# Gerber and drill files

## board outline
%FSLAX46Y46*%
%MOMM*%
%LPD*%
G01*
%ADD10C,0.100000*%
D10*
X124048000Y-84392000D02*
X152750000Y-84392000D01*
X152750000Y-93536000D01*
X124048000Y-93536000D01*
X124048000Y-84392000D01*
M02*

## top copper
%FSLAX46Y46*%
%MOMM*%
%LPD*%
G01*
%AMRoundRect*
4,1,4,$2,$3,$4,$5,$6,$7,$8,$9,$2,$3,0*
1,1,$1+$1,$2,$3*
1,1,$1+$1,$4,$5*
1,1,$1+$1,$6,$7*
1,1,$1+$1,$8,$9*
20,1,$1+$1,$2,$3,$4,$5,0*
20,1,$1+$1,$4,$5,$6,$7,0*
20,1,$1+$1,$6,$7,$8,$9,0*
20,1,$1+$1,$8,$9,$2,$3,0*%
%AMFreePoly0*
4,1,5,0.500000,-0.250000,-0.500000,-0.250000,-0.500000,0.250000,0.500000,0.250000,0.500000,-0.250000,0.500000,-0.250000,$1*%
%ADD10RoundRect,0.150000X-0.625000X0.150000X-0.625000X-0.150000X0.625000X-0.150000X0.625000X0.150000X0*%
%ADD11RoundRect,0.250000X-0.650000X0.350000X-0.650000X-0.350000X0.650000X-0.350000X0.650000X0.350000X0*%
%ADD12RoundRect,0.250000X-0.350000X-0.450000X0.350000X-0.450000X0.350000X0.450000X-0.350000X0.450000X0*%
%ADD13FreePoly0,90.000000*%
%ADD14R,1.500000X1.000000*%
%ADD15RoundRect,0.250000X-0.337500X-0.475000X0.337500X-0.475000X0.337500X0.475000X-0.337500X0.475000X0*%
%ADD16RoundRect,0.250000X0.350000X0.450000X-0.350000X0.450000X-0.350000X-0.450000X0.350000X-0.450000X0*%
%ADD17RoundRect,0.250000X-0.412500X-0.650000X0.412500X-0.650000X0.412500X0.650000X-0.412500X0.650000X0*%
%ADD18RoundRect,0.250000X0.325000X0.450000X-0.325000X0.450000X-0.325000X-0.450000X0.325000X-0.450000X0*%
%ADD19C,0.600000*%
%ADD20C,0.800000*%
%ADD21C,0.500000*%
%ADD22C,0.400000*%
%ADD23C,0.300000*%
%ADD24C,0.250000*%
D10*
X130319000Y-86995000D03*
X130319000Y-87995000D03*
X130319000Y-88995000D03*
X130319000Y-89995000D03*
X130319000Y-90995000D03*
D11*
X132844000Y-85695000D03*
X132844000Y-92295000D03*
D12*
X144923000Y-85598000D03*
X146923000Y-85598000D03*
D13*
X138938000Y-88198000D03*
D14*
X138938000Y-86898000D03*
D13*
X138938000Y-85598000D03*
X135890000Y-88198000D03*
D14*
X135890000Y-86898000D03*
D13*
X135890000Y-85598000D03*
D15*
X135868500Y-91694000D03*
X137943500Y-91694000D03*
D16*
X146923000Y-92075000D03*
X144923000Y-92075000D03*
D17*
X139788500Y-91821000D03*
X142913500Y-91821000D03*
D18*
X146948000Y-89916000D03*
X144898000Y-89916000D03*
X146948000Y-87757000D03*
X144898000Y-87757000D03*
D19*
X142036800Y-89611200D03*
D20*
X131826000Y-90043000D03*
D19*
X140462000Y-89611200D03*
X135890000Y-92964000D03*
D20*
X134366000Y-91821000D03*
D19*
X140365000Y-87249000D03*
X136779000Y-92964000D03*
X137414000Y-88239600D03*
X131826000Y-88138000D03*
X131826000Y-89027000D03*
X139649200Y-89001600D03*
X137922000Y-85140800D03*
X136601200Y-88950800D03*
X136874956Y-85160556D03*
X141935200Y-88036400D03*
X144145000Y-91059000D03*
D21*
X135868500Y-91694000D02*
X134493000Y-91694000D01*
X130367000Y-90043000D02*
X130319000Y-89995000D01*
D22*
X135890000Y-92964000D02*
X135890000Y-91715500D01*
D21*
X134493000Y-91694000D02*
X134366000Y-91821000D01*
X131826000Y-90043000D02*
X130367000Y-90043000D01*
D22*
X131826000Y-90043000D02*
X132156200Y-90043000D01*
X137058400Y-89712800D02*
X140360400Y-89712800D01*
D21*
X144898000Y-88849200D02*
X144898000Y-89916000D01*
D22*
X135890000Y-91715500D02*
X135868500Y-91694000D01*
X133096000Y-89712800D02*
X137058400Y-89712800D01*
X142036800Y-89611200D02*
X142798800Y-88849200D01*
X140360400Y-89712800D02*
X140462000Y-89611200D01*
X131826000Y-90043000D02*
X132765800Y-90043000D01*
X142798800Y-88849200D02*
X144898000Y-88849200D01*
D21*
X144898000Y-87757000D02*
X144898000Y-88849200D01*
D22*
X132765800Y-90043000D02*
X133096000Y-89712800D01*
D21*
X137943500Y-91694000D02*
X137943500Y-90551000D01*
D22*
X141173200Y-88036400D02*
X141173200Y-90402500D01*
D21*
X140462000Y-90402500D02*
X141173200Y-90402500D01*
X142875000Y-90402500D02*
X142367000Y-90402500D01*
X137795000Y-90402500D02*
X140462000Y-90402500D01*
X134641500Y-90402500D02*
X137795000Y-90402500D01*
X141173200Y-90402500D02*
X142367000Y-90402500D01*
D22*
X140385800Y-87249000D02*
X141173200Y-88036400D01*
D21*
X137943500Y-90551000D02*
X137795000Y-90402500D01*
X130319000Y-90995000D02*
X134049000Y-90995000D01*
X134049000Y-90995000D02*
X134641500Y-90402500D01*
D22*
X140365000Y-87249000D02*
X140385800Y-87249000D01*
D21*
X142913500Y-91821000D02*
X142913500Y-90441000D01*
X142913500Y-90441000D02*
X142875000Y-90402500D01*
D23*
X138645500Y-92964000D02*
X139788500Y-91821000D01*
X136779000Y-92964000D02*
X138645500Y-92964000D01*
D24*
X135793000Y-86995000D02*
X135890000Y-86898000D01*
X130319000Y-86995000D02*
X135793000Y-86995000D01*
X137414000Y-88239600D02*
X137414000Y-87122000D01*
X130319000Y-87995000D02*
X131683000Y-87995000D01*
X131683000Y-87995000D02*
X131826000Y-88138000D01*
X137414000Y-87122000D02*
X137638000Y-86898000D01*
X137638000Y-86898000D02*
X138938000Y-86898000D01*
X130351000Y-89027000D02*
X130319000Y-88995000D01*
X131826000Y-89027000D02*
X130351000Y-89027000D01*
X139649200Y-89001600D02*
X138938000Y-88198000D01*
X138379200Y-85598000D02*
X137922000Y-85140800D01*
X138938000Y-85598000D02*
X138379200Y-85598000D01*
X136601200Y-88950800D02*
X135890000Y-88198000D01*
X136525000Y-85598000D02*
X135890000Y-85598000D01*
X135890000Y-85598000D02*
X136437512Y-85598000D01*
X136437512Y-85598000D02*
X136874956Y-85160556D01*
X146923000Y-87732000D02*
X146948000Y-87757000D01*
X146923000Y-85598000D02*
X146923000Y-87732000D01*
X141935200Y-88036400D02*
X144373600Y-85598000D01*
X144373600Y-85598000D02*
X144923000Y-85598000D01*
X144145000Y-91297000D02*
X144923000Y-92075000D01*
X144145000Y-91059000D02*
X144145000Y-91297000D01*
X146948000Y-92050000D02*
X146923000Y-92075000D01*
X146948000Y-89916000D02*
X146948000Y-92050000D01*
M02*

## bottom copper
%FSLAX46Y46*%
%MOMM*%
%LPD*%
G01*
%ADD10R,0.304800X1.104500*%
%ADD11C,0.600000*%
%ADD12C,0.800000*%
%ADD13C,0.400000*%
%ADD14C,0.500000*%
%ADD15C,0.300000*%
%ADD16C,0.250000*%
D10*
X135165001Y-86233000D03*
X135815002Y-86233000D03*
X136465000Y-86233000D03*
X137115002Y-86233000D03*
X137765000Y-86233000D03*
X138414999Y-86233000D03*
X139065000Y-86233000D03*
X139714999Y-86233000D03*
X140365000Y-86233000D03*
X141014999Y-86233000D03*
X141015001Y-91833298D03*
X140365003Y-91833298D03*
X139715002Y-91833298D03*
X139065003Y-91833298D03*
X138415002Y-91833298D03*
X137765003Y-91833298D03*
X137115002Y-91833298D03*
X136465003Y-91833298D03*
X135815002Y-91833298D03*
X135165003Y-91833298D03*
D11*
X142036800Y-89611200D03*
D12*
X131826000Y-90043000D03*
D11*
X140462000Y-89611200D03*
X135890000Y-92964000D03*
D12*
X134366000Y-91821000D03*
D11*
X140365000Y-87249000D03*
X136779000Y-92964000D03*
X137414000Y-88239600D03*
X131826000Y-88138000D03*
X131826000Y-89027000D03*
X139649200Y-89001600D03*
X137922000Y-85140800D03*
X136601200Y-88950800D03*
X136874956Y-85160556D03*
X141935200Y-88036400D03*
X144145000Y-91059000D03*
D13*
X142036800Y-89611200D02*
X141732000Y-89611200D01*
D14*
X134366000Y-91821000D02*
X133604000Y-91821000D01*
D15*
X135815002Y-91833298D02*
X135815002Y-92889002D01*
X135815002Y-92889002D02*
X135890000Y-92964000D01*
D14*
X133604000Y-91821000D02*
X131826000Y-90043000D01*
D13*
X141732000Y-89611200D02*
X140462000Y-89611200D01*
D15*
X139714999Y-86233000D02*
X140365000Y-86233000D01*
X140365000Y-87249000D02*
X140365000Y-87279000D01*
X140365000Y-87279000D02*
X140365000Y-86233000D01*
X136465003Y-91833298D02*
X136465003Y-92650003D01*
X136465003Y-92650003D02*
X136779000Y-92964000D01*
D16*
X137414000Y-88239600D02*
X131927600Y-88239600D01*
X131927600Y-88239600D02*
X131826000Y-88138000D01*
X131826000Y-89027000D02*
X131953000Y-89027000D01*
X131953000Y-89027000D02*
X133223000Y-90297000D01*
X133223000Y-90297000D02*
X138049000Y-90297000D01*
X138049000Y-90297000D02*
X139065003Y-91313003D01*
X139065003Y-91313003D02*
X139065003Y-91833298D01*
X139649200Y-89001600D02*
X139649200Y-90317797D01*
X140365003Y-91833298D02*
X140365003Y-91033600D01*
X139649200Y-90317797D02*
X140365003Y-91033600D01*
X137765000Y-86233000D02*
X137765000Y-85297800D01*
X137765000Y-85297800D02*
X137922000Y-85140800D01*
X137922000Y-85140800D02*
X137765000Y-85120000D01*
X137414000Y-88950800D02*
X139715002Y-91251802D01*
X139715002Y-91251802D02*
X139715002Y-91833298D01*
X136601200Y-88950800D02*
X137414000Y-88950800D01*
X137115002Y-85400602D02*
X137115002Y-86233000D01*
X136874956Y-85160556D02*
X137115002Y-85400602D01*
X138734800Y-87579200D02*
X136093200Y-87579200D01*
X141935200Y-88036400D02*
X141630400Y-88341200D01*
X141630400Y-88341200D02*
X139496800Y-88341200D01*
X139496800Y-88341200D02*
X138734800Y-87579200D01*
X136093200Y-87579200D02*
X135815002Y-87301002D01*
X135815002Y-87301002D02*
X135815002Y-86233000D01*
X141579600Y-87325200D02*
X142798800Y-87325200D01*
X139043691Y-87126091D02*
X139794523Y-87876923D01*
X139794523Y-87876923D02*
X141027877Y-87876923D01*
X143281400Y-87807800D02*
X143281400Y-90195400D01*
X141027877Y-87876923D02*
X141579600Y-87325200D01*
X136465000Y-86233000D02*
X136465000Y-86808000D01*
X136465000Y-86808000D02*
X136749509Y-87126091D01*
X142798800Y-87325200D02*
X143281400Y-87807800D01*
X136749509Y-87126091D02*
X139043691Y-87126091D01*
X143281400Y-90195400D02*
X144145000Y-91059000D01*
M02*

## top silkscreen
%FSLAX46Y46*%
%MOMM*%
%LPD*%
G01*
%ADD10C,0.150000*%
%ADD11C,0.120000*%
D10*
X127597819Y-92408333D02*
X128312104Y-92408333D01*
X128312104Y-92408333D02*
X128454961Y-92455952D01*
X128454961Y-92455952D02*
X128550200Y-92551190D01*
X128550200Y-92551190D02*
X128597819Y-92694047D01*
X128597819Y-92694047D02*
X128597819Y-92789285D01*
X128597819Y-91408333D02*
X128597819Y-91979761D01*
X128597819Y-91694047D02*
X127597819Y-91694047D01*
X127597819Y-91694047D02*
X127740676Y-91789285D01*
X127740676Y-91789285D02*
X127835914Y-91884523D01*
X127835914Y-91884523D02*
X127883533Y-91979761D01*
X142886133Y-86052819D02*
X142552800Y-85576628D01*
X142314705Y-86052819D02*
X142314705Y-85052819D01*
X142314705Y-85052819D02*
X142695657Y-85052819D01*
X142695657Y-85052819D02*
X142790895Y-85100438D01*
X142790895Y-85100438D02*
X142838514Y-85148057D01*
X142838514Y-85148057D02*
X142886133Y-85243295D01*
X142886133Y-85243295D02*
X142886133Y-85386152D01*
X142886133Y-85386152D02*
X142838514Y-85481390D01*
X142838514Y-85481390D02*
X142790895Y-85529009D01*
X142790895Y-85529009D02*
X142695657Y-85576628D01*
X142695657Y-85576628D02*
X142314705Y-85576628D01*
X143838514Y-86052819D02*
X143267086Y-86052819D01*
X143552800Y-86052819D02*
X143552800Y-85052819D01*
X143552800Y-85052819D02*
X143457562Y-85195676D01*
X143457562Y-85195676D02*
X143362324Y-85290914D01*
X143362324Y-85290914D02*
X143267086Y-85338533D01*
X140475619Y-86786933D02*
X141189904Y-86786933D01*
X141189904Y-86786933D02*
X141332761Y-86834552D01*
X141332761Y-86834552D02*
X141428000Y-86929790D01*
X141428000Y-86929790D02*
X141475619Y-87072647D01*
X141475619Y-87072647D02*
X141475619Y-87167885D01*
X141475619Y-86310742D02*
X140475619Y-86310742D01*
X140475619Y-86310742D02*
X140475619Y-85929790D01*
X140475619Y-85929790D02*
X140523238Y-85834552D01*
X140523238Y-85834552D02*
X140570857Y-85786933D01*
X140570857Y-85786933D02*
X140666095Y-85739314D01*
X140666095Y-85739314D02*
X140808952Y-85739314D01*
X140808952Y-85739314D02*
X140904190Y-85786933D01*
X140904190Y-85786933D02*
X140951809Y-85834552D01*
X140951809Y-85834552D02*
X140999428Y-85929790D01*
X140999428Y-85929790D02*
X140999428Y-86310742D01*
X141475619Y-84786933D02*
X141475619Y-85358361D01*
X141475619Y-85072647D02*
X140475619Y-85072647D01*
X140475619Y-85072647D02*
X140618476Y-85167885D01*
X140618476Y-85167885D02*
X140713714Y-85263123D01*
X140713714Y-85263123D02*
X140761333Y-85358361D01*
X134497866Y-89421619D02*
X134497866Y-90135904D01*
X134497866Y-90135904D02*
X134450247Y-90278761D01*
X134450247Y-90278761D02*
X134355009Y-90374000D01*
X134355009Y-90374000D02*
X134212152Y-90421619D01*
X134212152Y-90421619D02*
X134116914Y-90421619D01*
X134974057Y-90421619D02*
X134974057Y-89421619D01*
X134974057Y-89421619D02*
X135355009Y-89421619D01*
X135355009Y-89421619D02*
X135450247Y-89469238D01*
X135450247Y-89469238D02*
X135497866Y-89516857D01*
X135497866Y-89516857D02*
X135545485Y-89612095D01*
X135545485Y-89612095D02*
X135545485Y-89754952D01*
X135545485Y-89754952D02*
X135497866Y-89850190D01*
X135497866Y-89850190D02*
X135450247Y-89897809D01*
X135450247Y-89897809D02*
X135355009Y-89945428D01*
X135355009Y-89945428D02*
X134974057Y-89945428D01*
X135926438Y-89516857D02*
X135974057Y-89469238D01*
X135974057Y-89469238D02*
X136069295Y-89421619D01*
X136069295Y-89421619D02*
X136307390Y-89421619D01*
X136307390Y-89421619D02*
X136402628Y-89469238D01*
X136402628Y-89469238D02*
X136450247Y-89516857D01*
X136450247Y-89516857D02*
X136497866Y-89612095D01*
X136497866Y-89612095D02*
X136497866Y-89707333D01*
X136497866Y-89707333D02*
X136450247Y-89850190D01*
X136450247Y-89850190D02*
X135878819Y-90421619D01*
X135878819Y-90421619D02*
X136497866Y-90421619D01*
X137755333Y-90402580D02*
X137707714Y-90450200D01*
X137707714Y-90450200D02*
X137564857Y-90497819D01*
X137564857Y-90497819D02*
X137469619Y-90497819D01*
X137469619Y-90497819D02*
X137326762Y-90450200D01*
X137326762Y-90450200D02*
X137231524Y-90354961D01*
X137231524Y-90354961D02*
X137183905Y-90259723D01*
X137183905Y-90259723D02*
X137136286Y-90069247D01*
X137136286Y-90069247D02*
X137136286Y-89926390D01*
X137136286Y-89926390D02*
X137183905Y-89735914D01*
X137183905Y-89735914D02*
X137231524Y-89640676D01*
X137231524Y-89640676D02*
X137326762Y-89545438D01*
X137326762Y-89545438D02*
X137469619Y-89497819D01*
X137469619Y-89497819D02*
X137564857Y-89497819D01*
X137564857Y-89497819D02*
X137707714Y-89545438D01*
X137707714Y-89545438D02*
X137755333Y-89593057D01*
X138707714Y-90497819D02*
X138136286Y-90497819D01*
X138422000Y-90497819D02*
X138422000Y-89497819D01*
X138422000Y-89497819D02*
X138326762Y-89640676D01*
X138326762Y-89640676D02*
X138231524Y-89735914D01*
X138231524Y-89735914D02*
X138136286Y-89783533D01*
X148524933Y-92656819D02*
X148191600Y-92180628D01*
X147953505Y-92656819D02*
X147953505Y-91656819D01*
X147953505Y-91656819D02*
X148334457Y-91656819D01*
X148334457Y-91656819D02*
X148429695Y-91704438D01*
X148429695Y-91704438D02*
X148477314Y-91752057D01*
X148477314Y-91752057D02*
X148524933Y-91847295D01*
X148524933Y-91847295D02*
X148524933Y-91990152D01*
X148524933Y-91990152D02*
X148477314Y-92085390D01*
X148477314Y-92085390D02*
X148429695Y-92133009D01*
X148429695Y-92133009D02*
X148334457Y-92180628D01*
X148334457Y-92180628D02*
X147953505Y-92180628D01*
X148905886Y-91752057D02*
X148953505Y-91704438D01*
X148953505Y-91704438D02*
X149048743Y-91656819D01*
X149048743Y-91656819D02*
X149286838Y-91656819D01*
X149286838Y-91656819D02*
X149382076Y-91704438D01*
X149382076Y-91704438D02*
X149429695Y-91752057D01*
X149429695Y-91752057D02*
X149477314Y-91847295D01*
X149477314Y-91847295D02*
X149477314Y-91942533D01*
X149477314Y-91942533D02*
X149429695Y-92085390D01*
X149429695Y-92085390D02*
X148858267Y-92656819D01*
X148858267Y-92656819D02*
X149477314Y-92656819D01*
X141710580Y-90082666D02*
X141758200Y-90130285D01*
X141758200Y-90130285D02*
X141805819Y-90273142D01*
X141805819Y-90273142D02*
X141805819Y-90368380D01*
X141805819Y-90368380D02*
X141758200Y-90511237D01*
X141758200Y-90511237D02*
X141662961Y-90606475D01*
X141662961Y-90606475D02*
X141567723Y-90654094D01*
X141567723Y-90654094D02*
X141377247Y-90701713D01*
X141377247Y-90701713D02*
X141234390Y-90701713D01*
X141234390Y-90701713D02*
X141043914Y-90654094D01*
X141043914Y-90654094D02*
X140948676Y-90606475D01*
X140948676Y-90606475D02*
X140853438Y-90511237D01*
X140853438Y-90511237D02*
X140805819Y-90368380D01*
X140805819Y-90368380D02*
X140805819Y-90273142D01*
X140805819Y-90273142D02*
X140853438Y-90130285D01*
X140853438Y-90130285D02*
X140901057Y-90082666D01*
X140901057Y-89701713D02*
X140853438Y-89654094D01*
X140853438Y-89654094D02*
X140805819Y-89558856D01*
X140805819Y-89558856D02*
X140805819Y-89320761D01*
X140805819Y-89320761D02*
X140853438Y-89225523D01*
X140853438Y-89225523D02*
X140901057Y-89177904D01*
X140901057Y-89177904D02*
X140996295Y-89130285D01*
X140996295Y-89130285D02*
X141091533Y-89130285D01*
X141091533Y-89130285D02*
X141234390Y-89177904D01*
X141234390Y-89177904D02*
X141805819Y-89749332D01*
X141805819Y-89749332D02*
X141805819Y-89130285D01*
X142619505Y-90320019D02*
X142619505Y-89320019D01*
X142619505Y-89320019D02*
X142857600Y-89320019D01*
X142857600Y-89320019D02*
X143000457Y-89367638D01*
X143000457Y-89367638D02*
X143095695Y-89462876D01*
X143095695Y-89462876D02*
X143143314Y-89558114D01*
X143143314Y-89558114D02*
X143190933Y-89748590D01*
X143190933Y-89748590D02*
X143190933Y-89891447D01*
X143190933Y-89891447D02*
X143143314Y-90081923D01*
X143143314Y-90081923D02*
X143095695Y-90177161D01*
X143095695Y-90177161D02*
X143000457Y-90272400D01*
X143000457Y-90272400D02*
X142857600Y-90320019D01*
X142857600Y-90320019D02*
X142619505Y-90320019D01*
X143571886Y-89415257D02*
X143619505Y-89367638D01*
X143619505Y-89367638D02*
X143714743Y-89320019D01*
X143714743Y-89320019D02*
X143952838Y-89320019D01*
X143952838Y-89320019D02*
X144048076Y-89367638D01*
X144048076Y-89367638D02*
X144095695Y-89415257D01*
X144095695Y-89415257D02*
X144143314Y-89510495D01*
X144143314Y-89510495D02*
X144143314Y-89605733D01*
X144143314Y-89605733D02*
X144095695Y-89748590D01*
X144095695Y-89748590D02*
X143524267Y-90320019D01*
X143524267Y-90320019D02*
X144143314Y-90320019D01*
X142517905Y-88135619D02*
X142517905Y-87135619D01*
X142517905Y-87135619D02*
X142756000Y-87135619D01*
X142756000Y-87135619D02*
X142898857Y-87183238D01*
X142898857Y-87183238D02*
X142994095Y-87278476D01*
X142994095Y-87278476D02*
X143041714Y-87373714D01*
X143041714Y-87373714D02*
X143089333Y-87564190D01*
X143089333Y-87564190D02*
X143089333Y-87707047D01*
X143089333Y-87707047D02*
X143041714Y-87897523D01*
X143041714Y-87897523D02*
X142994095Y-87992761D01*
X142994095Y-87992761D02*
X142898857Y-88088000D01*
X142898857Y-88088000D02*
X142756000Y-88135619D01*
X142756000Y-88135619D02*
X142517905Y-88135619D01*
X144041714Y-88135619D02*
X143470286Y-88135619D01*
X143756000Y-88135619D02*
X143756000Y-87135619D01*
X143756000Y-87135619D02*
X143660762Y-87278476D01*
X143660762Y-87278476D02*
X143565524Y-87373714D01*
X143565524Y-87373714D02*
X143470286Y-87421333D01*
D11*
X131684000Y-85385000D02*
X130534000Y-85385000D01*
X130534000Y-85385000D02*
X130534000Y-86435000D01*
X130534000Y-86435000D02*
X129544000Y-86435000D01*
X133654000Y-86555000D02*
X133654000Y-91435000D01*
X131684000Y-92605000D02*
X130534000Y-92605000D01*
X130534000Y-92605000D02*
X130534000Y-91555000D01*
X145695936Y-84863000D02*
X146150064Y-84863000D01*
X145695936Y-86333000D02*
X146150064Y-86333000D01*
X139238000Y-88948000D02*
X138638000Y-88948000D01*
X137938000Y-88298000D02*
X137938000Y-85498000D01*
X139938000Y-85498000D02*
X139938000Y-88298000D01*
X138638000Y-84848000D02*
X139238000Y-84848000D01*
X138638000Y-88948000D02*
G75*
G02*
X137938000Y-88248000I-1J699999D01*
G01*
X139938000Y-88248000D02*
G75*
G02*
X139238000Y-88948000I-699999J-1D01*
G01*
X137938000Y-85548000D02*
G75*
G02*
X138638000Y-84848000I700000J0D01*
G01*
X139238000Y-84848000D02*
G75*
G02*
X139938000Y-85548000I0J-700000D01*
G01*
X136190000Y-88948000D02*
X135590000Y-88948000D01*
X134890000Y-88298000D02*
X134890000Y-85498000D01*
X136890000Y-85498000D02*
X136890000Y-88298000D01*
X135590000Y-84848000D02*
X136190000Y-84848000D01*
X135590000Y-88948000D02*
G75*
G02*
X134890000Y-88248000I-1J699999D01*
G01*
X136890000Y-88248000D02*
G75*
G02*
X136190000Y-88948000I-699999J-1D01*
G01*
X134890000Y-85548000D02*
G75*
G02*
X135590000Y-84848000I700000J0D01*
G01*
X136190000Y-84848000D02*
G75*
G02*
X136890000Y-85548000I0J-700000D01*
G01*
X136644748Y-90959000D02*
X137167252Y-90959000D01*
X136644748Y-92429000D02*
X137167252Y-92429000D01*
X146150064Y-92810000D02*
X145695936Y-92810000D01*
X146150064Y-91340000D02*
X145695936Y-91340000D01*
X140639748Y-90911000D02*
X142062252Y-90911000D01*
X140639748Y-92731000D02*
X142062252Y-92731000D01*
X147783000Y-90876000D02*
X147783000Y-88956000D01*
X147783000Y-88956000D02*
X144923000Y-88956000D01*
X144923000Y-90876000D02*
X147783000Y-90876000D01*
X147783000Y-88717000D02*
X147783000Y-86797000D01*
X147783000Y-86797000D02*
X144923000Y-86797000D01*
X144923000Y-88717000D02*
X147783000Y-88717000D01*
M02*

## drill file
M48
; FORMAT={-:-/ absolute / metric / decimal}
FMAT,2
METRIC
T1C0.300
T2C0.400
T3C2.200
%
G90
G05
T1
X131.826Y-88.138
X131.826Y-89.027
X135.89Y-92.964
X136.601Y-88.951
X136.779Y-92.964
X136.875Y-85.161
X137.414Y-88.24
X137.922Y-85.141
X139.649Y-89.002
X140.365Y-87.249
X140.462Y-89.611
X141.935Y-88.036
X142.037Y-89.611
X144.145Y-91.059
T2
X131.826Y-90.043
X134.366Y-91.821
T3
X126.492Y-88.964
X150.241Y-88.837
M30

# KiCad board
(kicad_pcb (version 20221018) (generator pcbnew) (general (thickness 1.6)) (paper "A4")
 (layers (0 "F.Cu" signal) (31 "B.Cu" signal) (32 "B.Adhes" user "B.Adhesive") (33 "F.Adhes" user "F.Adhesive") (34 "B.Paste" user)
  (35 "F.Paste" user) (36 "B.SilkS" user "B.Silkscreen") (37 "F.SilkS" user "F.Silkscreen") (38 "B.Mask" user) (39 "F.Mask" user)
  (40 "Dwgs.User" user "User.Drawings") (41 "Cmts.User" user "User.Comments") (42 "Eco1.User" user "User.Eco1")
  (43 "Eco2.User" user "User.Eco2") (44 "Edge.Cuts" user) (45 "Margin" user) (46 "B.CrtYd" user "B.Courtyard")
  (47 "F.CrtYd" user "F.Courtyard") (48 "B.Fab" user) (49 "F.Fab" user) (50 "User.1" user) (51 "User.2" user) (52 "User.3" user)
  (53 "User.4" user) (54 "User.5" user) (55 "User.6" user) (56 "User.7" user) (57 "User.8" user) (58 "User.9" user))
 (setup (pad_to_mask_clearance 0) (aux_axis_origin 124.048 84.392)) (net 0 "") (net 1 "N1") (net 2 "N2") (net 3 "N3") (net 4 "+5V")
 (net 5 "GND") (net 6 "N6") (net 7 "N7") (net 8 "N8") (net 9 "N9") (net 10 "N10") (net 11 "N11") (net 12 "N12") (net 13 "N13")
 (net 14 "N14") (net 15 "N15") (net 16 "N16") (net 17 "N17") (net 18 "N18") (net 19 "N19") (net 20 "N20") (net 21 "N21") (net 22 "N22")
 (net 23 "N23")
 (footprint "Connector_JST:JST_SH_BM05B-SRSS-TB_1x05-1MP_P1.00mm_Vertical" (layer "F.Cu") (at 131.644 88.995 -90)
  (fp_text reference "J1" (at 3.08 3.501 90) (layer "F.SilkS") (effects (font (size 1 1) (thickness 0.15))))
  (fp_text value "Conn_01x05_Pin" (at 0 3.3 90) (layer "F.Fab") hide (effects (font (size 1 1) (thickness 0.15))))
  (fp_line (start -3.61 -0.04) (end -3.61 1.11) (stroke (width 0.12) (type solid)) (layer "F.SilkS"))
  (fp_line (start -3.61 1.11) (end -2.56 1.11) (stroke (width 0.12) (type solid)) (layer "F.SilkS"))
  (fp_line (start -2.56 1.11) (end -2.56 2.1) (stroke (width 0.12) (type solid)) (layer "F.SilkS"))
  (fp_line (start -2.44 -2.01) (end 2.44 -2.01) (stroke (width 0.12) (type solid)) (layer "F.SilkS"))
  (fp_line (start 3.61 -0.04) (end 3.61 1.11) (stroke (width 0.12) (type solid)) (layer "F.SilkS"))
  (fp_line (start 3.61 1.11) (end 2.56 1.11) (stroke (width 0.12) (type solid)) (layer "F.SilkS"))
  (pad "1" smd roundrect (at -2 1.325 270) (size 0.6 1.55) (layers "F.Cu" "F.Paste" "F.Mask") (roundrect_rratio 0.25) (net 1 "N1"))
  (pad "2" smd roundrect (at -1 1.325 270) (size 0.6 1.55) (layers "F.Cu" "F.Paste" "F.Mask") (roundrect_rratio 0.25) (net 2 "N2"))
  (pad "3" smd roundrect (at 0 1.325 270) (size 0.6 1.55) (layers "F.Cu" "F.Paste" "F.Mask") (roundrect_rratio 0.25) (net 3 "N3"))
  (pad "4" smd roundrect (at 1 1.325 270) (size 0.6 1.55) (layers "F.Cu" "F.Paste" "F.Mask") (roundrect_rratio 0.25) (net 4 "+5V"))
  (pad "5" smd roundrect (at 2 1.325 270) (size 0.6 1.55) (layers "F.Cu" "F.Paste" "F.Mask") (roundrect_rratio 0.25) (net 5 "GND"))
  (pad "MP" smd roundrect (at -3.3 -1.2 270) (size 1.2 1.8) (layers "F.Cu" "F.Paste" "F.Mask") (roundrect_rratio 0.2083333333))
  (pad "MP" smd roundrect (at 3.3 -1.2 270) (size 1.2 1.8) (layers "F.Cu" "F.Paste" "F.Mask") (roundrect_rratio 0.2083333333)))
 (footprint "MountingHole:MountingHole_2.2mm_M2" (layer "F.Cu") (at 126.492 88.964 90)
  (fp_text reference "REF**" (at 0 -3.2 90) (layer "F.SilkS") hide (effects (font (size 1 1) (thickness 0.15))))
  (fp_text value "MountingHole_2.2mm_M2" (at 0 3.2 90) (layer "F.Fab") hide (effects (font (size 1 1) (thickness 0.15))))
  (pad "" np_thru_hole circle (at 0 0 90) (size 2.2 2.2) (drill 2.2) (layers "F&B.Cu" "*.Mask")))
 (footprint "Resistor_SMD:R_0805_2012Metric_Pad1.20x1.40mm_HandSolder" (layer "F.Cu") (at 145.923 85.598)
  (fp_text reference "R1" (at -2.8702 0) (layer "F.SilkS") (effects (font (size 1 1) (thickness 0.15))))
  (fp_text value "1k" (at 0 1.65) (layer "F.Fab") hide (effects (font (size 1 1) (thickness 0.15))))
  (fp_line (start -0.227064 -0.735) (end 0.227064 -0.735) (stroke (width 0.12) (type solid)) (layer "F.SilkS"))
  (fp_line (start -0.227064 0.735) (end 0.227064 0.735) (stroke (width 0.12) (type solid)) (layer "F.SilkS"))
  (pad "1" smd roundrect (at -1 0) (size 1.2 1.4) (layers "F.Cu" "F.Paste" "F.Mask") (roundrect_rratio 0.2083333333) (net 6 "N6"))
  (pad "2" smd roundrect (at 1 0) (size 1.2 1.4) (layers "F.Cu" "F.Paste" "F.Mask") (roundrect_rratio 0.2083333333) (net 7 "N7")))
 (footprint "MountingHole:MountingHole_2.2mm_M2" (layer "F.Cu") (at 150.241 88.837 90)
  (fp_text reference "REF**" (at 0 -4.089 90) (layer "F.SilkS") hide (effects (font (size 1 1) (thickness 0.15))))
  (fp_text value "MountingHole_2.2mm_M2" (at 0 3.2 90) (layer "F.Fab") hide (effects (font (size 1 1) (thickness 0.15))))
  (pad "" np_thru_hole circle (at 0 0 90) (size 2.2 2.2) (drill 2.2) (layers "*.Cu" "*.Mask")))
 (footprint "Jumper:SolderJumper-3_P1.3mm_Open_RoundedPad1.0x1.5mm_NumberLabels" (layer "F.Cu") (at 138.938 86.898 90)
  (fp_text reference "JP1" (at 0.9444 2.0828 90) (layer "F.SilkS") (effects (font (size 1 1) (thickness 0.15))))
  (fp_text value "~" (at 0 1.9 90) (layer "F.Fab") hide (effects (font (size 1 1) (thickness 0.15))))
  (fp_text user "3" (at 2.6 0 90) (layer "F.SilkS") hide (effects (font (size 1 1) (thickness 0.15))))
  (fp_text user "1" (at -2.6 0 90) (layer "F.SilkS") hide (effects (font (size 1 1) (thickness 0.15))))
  (fp_line (start -2.05 0.3) (end -2.05 -0.3) (stroke (width 0.12) (type solid)) (layer "F.SilkS"))
  (fp_line (start -1.4 -1) (end 1.4 -1) (stroke (width 0.12) (type solid)) (layer "F.SilkS"))
  (fp_line (start 1.4 1) (end -1.4 1) (stroke (width 0.12) (type solid)) (layer "F.SilkS"))
  (fp_line (start 2.05 -0.3) (end 2.05 0.3) (stroke (width 0.12) (type solid)) (layer "F.SilkS"))
  (fp_arc (start -2.05 -0.3) (mid -1.844975 -0.794975) (end -1.35 -1) (stroke (width 0.12) (type solid)) (layer "F.SilkS"))
  (fp_arc (start -1.35 1) (mid -1.844975 0.794975) (end -2.05 0.3) (stroke (width 0.12) (type solid)) (layer "F.SilkS"))
  (fp_arc (start 1.35 -1) (mid 1.844975 -0.794975) (end 2.05 -0.3) (stroke (width 0.12) (type solid)) (layer "F.SilkS"))
  (fp_arc (start 2.05 0.3) (mid 1.844975 0.794975) (end 1.35 1) (stroke (width 0.12) (type solid)) (layer "F.SilkS"))
  (pad "1" smd custom (at -1.3 0 90) (size 1 0.5) (layers "F.Cu" "F.Mask") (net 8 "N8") (zone_connect 2)
   (options (clearance outline) (anchor rect)) (primitives))
  (pad "2" smd rect (at 0 0 90) (size 1 1.5) (layers "F.Cu" "F.Mask") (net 2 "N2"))
  (pad "3" smd custom (at 1.3 0 90) (size 1 0.5) (layers "F.Cu" "F.Mask") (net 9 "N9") (zone_connect 2)
   (options (clearance outline) (anchor rect)) (primitives)))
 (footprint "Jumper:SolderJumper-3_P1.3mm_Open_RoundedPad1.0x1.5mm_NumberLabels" (layer "F.Cu") (at 135.89 86.898 90)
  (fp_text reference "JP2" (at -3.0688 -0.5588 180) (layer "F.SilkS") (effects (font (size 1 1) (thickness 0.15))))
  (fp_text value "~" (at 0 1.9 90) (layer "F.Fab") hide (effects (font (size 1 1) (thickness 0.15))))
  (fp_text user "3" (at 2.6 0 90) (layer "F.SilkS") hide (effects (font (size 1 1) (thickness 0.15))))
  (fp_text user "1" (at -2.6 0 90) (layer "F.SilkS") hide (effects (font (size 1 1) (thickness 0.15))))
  (fp_line (start -2.05 0.3) (end -2.05 -0.3) (stroke (width 0.12) (type solid)) (layer "F.SilkS"))
  (fp_line (start -1.4 -1) (end 1.4 -1) (stroke (width 0.12) (type solid)) (layer "F.SilkS"))
  (fp_line (start 1.4 1) (end -1.4 1) (stroke (width 0.12) (type solid)) (layer "F.SilkS"))
  (fp_line (start 2.05 -0.3) (end 2.05 0.3) (stroke (width 0.12) (type solid)) (layer "F.SilkS"))
  (fp_arc (start -2.05 -0.3) (mid -1.844975 -0.794975) (end -1.35 -1) (stroke (width 0.12) (type solid)) (layer "F.SilkS"))
  (fp_arc (start -1.35 1) (mid -1.844975 0.794975) (end -2.05 0.3) (stroke (width 0.12) (type solid)) (layer "F.SilkS"))
  (fp_arc (start 1.35 -1) (mid 1.844975 -0.794975) (end 2.05 -0.3) (stroke (width 0.12) (type solid)) (layer "F.SilkS"))
  (fp_arc (start 2.05 0.3) (mid 1.844975 0.794975) (end 1.35 1) (stroke (width 0.12) (type solid)) (layer "F.SilkS"))
  (pad "1" smd custom (at -1.3 0 90) (size 1 0.5) (layers "F.Cu" "F.Mask") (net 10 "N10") (zone_connect 2)
   (options (clearance outline) (anchor rect)) (primitives))
  (pad "2" smd rect (at 0 0 90) (size 1 1.5) (layers "F.Cu" "F.Mask") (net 1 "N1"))
  (pad "3" smd custom (at 1.3 0 90) (size 1 0.5) (layers "F.Cu" "F.Mask") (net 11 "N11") (zone_connect 2)
   (options (clearance outline) (anchor rect)) (primitives)))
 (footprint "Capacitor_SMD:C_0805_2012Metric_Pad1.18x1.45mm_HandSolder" (layer "F.Cu") (at 136.906 91.694)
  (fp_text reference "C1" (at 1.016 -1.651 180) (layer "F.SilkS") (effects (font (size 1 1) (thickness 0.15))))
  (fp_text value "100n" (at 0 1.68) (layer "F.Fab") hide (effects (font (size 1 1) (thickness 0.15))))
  (fp_line (start -0.261252 -0.735) (end 0.261252 -0.735) (stroke (width 0.12) (type solid)) (layer "F.SilkS"))
  (fp_line (start -0.261252 0.735) (end 0.261252 0.735) (stroke (width 0.12) (type solid)) (layer "F.SilkS"))
  (pad "1" smd roundrect (at -1.0375 0) (size 1.175 1.45) (layers "F.Cu" "F.Paste" "F.Mask") (roundrect_rratio 0.2127659574) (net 4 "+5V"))
  (pad "2" smd roundrect (at 1.0375 0) (size 1.175 1.45) (layers "F.Cu" "F.Paste" "F.Mask") (roundrect_rratio 0.2127659574) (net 5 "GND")))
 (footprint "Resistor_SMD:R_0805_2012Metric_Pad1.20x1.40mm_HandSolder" (layer "F.Cu") (at 145.923 92.075 180)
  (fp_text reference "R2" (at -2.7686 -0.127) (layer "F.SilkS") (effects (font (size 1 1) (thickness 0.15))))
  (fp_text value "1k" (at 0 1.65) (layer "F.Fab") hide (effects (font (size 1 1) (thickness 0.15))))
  (fp_line (start -0.227064 -0.735) (end 0.227064 -0.735) (stroke (width 0.12) (type solid)) (layer "F.SilkS"))
  (fp_line (start -0.227064 0.735) (end 0.227064 0.735) (stroke (width 0.12) (type solid)) (layer "F.SilkS"))
  (pad "1" smd roundrect (at -1 0 180) (size 1.2 1.4) (layers "F.Cu" "F.Paste" "F.Mask") (roundrect_rratio 0.2083333333) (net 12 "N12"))
  (pad "2" smd roundrect (at 1 0 180) (size 1.2 1.4) (layers "F.Cu" "F.Paste" "F.Mask") (roundrect_rratio 0.2083333333) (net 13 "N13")))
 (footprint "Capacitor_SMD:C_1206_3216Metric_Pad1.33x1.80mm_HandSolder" (layer "F.Cu") (at 141.351 91.821)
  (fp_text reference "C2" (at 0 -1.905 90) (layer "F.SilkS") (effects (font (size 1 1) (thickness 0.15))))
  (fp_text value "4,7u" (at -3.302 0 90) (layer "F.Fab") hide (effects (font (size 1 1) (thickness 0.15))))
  (fp_line (start -0.711252 -0.91) (end 0.711252 -0.91) (stroke (width 0.12) (type solid)) (layer "F.SilkS"))
  (fp_line (start -0.711252 0.91) (end 0.711252 0.91) (stroke (width 0.12) (type solid)) (layer "F.SilkS"))
  (pad "1" smd roundrect (at -1.5625 0) (size 1.325 1.8) (layers "F.Cu" "F.Paste" "F.Mask") (roundrect_rratio 0.1886792453) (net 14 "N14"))
  (pad "2" smd roundrect (at 1.5625 0) (size 1.325 1.8) (layers "F.Cu" "F.Paste" "F.Mask") (roundrect_rratio 0.1886792453) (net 5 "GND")))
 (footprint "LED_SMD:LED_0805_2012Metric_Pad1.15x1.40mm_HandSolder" (layer "F.Cu") (at 145.923 89.916 180)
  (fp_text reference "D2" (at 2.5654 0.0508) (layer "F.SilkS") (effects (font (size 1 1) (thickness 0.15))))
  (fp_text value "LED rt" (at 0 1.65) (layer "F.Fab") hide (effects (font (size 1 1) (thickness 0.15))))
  (fp_line (start -1.86 -0.96) (end -1.86 0.96) (stroke (width 0.12) (type solid)) (layer "F.SilkS"))
  (fp_line (start -1.86 0.96) (end 1 0.96) (stroke (width 0.12) (type solid)) (layer "F.SilkS"))
  (fp_line (start 1 -0.96) (end -1.86 -0.96) (stroke (width 0.12) (type solid)) (layer "F.SilkS"))
  (pad "1" smd roundrect (at -1.025 0 180) (size 1.15 1.4) (layers "F.Cu" "F.Paste" "F.Mask") (roundrect_rratio 0.2173913043) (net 12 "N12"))
  (pad "2" smd roundrect (at 1.025 0 180) (size 1.15 1.4) (layers "F.Cu" "F.Paste" "F.Mask") (roundrect_rratio 0.2173913043) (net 4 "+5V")))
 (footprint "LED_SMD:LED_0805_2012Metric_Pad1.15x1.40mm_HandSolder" (layer "F.Cu") (at 145.923 87.757 180)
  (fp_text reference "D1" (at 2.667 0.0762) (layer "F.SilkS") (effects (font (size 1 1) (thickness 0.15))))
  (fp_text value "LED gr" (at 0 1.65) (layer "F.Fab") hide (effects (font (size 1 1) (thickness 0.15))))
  (fp_line (start -1.86 -0.96) (end -1.86 0.96) (stroke (width 0.12) (type solid)) (layer "F.SilkS"))
  (fp_line (start -1.86 0.96) (end 1 0.96) (stroke (width 0.12) (type solid)) (layer "F.SilkS"))
  (fp_line (start 1 -0.96) (end -1.86 -0.96) (stroke (width 0.12) (type solid)) (layer "F.SilkS"))
  (pad "1" smd roundrect (at -1.025 0 180) (size 1.15 1.4) (layers "F.Cu" "F.Paste" "F.Mask") (roundrect_rratio 0.2173913043) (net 7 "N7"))
  (pad "2" smd roundrect (at 1.025 0 180) (size 1.15 1.4) (layers "F.Cu" "F.Paste" "F.Mask") (roundrect_rratio 0.2173913043) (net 4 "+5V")))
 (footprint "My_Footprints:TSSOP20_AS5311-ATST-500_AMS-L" (layer "B.Cu") (at 138.090001 89.033149 -90)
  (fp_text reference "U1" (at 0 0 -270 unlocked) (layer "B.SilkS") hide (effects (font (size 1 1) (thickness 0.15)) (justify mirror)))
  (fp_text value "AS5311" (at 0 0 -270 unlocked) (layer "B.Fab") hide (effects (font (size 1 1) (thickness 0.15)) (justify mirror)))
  (pad "1" smd rect (at -2.800149 2.925 270) (size 1.1045 0.3048) (layers "B.Cu" "B.Paste" "B.Mask") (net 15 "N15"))
  (pad "2" smd rect (at -2.800149 2.274999 270) (size 1.1045 0.3048) (layers "B.Cu" "B.Paste" "B.Mask") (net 6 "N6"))
  (pad "3" smd rect (at -2.800149 1.625001 270) (size 1.1045 0.3048) (layers "B.Cu" "B.Paste" "B.Mask") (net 13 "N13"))
  (pad "4" smd rect (at -2.800149 0.974999 270) (size 1.1045 0.3048) (layers "B.Cu" "B.Paste" "B.Mask") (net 11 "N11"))
  (pad "5" smd rect (at -2.800149 0.325001 270) (size 1.1045 0.3048) (layers "B.Cu" "B.Paste" "B.Mask") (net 9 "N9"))
  (pad "6" smd rect (at -2.800149 -0.324998 270) (size 1.1045 0.3048) (layers "B.Cu" "B.Paste" "B.Mask") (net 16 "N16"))
  (pad "7" smd rect (at -2.800149 -0.974999 270) (size 1.1045 0.3048) (layers "B.Cu" "B.Paste" "B.Mask") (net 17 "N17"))
  (pad "8" smd rect (at -2.800149 -1.624998 270) (size 1.1045 0.3048) (layers "B.Cu" "B.Paste" "B.Mask") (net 5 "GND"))
  (pad "9" smd rect (at -2.800149 -2.274999 270) (size 1.1045 0.3048) (layers "B.Cu" "B.Paste" "B.Mask") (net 5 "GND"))
  (pad "10" smd rect (at -2.800149 -2.924998 270) (size 1.1045 0.3048) (layers "B.Cu" "B.Paste" "B.Mask") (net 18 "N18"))
  (pad "11" smd rect (at 2.800149 -2.925 270) (size 1.1045 0.3048) (layers "B.Cu" "B.Paste" "B.Mask") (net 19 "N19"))
  (pad "12" smd rect (at 2.800149 -2.275002 270) (size 1.1045 0.3048) (layers "B.Cu" "B.Paste" "B.Mask") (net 8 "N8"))
  (pad "13" smd rect (at 2.800149 -1.625001 270) (size 1.1045 0.3048) (layers "B.Cu" "B.Paste" "B.Mask") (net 10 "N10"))
  (pad "14" smd rect (at 2.800149 -0.975002 270) (size 1.1045 0.3048) (layers "B.Cu" "B.Paste" "B.Mask") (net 3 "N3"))
  (pad "15" smd rect (at 2.800149 -0.325001 270) (size 1.1045 0.3048) (layers "B.Cu" "B.Paste" "B.Mask") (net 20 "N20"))
  (pad "16" smd rect (at 2.800149 0.324998 270) (size 1.1045 0.3048) (layers "B.Cu" "B.Paste" "B.Mask") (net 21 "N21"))
  (pad "17" smd rect (at 2.800149 0.974999 270) (size 1.1045 0.3048) (layers "B.Cu" "B.Paste" "B.Mask") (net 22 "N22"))
  (pad "18" smd rect (at 2.800149 1.624998 270) (size 1.1045 0.3048) (layers "B.Cu" "B.Paste" "B.Mask") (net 14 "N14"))
  (pad "19" smd rect (at 2.800149 2.274999 270) (size 1.1045 0.3048) (layers "B.Cu" "B.Paste" "B.Mask") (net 4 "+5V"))
  (pad "20" smd rect (at 2.800149 2.924998 270) (size 1.1045 0.3048) (layers "B.Cu" "B.Paste" "B.Mask") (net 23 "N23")))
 (gr_rect (start 124.048 84.392) (end 152.75 93.536) (stroke (width 0.1) (type default)) (fill none) (layer "Edge.Cuts"))
 (segment (start 135.8685 91.694) (end 134.493 91.694) (width 0.5) (layer "F.Cu") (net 4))
 (segment (start 130.367 90.043) (end 130.319 89.995) (width 0.5) (layer "F.Cu") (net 4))
 (segment (start 135.89 92.964) (end 135.89 91.7155) (width 0.4) (layer "F.Cu") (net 4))
 (segment (start 134.493 91.694) (end 134.366 91.821) (width 0.5) (layer "F.Cu") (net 4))
 (segment (start 131.826 90.043) (end 130.367 90.043) (width 0.5) (layer "F.Cu") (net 4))
 (segment (start 131.826 90.043) (end 132.1562 90.043) (width 0.4) (layer "F.Cu") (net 4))
 (segment (start 137.0584 89.7128) (end 140.3604 89.7128) (width 0.4) (layer "F.Cu") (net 4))
 (segment (start 144.898 88.8492) (end 144.898 89.916) (width 0.5) (layer "F.Cu") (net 4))
 (segment (start 135.89 91.7155) (end 135.8685 91.694) (width 0.4) (layer "F.Cu") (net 4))
 (segment (start 133.096 89.7128) (end 137.0584 89.7128) (width 0.4) (layer "F.Cu") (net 4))
 (segment (start 142.0368 89.6112) (end 142.7988 88.8492) (width 0.4) (layer "F.Cu") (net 4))
 (segment (start 140.3604 89.7128) (end 140.462 89.6112) (width 0.4) (layer "F.Cu") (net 4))
 (segment (start 131.826 90.043) (end 132.7658 90.043) (width 0.4) (layer "F.Cu") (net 4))
 (segment (start 142.7988 88.8492) (end 144.898 88.8492) (width 0.4) (layer "F.Cu") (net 4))
 (segment (start 144.898 87.757) (end 144.898 88.8492) (width 0.5) (layer "F.Cu") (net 4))
 (segment (start 132.7658 90.043) (end 133.096 89.7128) (width 0.4) (layer "F.Cu") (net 4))
 (via (at 142.0368 89.6112) (size 0.6) (drill 0.3) (layers "F.Cu" "B.Cu") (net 4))
 (via (at 131.826 90.043) (size 0.8) (drill 0.4) (layers "F.Cu" "B.Cu") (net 4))
 (via (at 140.462 89.6112) (size 0.6) (drill 0.3) (layers "F.Cu" "B.Cu") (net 4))
 (via (at 135.89 92.964) (size 0.6) (drill 0.3) (layers "F.Cu" "B.Cu") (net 4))
 (via (at 134.366 91.821) (size 0.8) (drill 0.4) (layers "F.Cu" "B.Cu") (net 4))
 (segment (start 142.0368 89.6112) (end 141.732 89.6112) (width 0.4) (layer "B.Cu") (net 4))
 (segment (start 134.366 91.821) (end 133.604 91.821) (width 0.5) (layer "B.Cu") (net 4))
 (segment (start 135.815002 91.833298) (end 135.815002 92.889002) (width 0.3) (layer "B.Cu") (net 4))
 (segment (start 135.815002 92.889002) (end 135.89 92.964) (width 0.3) (layer "B.Cu") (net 4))
 (segment (start 133.604 91.821) (end 131.826 90.043) (width 0.5) (layer "B.Cu") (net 4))
 (segment (start 141.732 89.6112) (end 140.462 89.6112) (width 0.4) (layer "B.Cu") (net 4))
 (segment (start 137.9435 91.694) (end 137.9435 90.551) (width 0.5) (layer "F.Cu") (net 5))
 (segment (start 141.1732 88.0364) (end 141.1732 90.4025) (width 0.4) (layer "F.Cu") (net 5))
 (segment (start 140.462 90.4025) (end 141.1732 90.4025) (width 0.5) (layer "F.Cu") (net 5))
 (segment (start 142.875 90.4025) (end 142.367 90.4025) (width 0.5) (layer "F.Cu") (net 5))
 (segment (start 137.795 90.4025) (end 140.462 90.4025) (width 0.5) (layer "F.Cu") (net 5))
 (segment (start 134.6415 90.4025) (end 137.795 90.4025) (width 0.5) (layer "F.Cu") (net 5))
 (segment (start 141.1732 90.4025) (end 142.367 90.4025) (width 0.5) (layer "F.Cu") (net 5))
 (segment (start 140.3858 87.249) (end 141.1732 88.0364) (width 0.4) (layer "F.Cu") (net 5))
 (segment (start 137.9435 90.551) (end 137.795 90.4025) (width 0.5) (layer "F.Cu") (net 5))
 (segment (start 130.319 90.995) (end 134.049 90.995) (width 0.5) (layer "F.Cu") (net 5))
 (segment (start 134.049 90.995) (end 134.6415 90.4025) (width 0.5) (layer "F.Cu") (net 5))
 (segment (start 140.365 87.249) (end 140.3858 87.249) (width 0.4) (layer "F.Cu") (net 5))
 (segment (start 142.9135 91.821) (end 142.9135 90.441) (width 0.5) (layer "F.Cu") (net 5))
 (segment (start 142.9135 90.441) (end 142.875 90.4025) (width 0.5) (layer "F.Cu") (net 5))
 (via (at 140.365 87.249) (size 0.6) (drill 0.3) (layers "F.Cu" "B.Cu") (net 5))
 (segment (start 139.714999 86.233) (end 140.365 86.233) (width 0.3) (layer "B.Cu") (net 5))
 (segment (start 140.365 87.249) (end 140.365 87.279) (width 0.3) (layer "B.Cu") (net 5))
 (segment (start 140.365 87.279) (end 140.365 86.233) (width 0.3) (layer "B.Cu") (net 5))
 (segment (start 138.6455 92.964) (end 139.7885 91.821) (width 0.3) (layer "F.Cu") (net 14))
 (segment (start 136.779 92.964) (end 138.6455 92.964) (width 0.3) (layer "F.Cu") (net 14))
 (via (at 136.779 92.964) (size 0.6) (drill 0.3) (layers "F.Cu" "B.Cu") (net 14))
 (segment (start 136.465003 91.833298) (end 136.465003 92.650003) (width 0.3) (layer "B.Cu") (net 14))
 (segment (start 136.465003 92.650003) (end 136.779 92.964) (width 0.3) (layer "B.Cu") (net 14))
 (segment (start 135.793 86.995) (end 135.89 86.898) (width 0.25) (layer "F.Cu") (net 1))
 (segment (start 130.319 86.995) (end 135.793 86.995) (width 0.25) (layer "F.Cu") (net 1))
 (segment (start 137.414 88.2396) (end 137.414 87.122) (width 0.25) (layer "F.Cu") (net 2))
 (segment (start 130.319 87.995) (end 131.683 87.995) (width 0.25) (layer "F.Cu") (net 2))
 (segment (start 131.683 87.995) (end 131.826 88.138) (width 0.25) (layer "F.Cu") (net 2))
 (segment (start 137.414 87.122) (end 137.638 86.898) (width 0.25) (layer "F.Cu") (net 2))
 (segment (start 137.638 86.898) (end 138.938 86.898) (width 0.25) (layer "F.Cu") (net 2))
 (via (at 137.414 88.2396) (size 0.6) (drill 0.3) (layers "F.Cu" "B.Cu") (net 2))
 (via (at 131.826 88.138) (size 0.6) (drill 0.3) (layers "F.Cu" "B.Cu") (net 2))
 (segment (start 137.414 88.2396) (end 131.9276 88.2396) (width 0.25) (layer "B.Cu") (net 2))
 (segment (start 131.9276 88.2396) (end 131.826 88.138) (width 0.25) (layer "B.Cu") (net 2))
 (segment (start 130.351 89.027) (end 130.319 88.995) (width 0.25) (layer "F.Cu") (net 3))
 (segment (start 131.826 89.027) (end 130.351 89.027) (width 0.25) (layer "F.Cu") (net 3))
 (via (at 131.826 89.027) (size 0.6) (drill 0.3) (layers "F.Cu" "B.Cu") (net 3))
 (segment (start 131.826 89.027) (end 131.953 89.027) (width 0.25) (layer "B.Cu") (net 3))
 (segment (start 131.953 89.027) (end 133.223 90.297) (width 0.25) (layer "B.Cu") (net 3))
 (segment (start 133.223 90.297) (end 138.049 90.297) (width 0.25) (layer "B.Cu") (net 3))
 (segment (start 138.049 90.297) (end 139.065003 91.313003) (width 0.25) (layer "B.Cu") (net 3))
 (segment (start 139.065003 91.313003) (end 139.065003 91.833298) (width 0.25) (layer "B.Cu") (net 3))
 (segment (start 139.6492 89.0016) (end 138.938 88.198) (width 0.25) (layer "F.Cu") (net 8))
 (via (at 139.6492 89.0016) (size 0.6) (drill 0.3) (layers "F.Cu" "B.Cu") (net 8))
 (segment (start 139.6492 89.0016) (end 139.6492 90.317797) (width 0.25) (layer "B.Cu") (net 8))
 (segment (start 140.365003 91.833298) (end 140.365003 91.0336) (width 0.25) (layer "B.Cu") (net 8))
 (segment (start 139.6492 90.317797) (end 140.365003 91.0336) (width 0.25) (layer "B.Cu") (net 8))
 (segment (start 138.3792 85.598) (end 137.922 85.1408) (width 0.25) (layer "F.Cu") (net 9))
 (segment (start 138.938 85.598) (end 138.3792 85.598) (width 0.25) (layer "F.Cu") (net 9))
 (via (at 137.922 85.1408) (size 0.6) (drill 0.3) (layers "F.Cu" "B.Cu") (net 9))
 (segment (start 137.765 86.233) (end 137.765 85.2978) (width 0.25) (layer "B.Cu") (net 9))
 (segment (start 137.765 85.2978) (end 137.922 85.1408) (width 0.25) (layer "B.Cu") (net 9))
 (segment (start 137.922 85.1408) (end 137.765 85.12) (width 0.25) (layer "B.Cu") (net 9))
 (segment (start 136.6012 88.9508) (end 135.89 88.198) (width 0.25) (layer "F.Cu") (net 10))
 (via (at 136.6012 88.9508) (size 0.6) (drill 0.3) (layers "F.Cu" "B.Cu") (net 10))
 (segment (start 137.414 88.9508) (end 139.715002 91.251802) (width 0.25) (layer "B.Cu") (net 10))
 (segment (start 139.715002 91.251802) (end 139.715002 91.833298) (width 0.25) (layer "B.Cu") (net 10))
 (segment (start 136.6012 88.9508) (end 137.414 88.9508) (width 0.25) (layer "B.Cu") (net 10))
 (segment (start 136.525 85.598) (end 135.89 85.598) (width 0.25) (layer "F.Cu") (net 11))
 (segment (start 135.89 85.598) (end 136.437512 85.598) (width 0.25) (layer "F.Cu") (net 11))
 (segment (start 136.437512 85.598) (end 136.874956 85.160556) (width 0.25) (layer "F.Cu") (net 11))
 (via (at 136.874956 85.160556) (size 0.6) (drill 0.3) (layers "F.Cu" "B.Cu") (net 11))
 (segment (start 137.115002 85.400602) (end 137.115002 86.233) (width 0.25) (layer "B.Cu") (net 11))
 (segment (start 136.874956 85.160556) (end 137.115002 85.400602) (width 0.25) (layer "B.Cu") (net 11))
 (segment (start 146.923 87.732) (end 146.948 87.757) (width 0.25) (layer "F.Cu") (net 7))
 (segment (start 146.923 85.598) (end 146.923 87.732) (width 0.25) (layer "F.Cu") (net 7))
 (segment (start 141.9352 88.0364) (end 144.3736 85.598) (width 0.25) (layer "F.Cu") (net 6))
 (segment (start 144.3736 85.598) (end 144.923 85.598) (width 0.25) (layer "F.Cu") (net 6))
 (via (at 141.9352 88.0364) (size 0.6) (drill 0.3) (layers "F.Cu" "B.Cu") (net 6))
 (segment (start 138.7348 87.5792) (end 136.0932 87.5792) (width 0.25) (layer "B.Cu") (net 6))
 (segment (start 141.9352 88.0364) (end 141.6304 88.3412) (width 0.25) (layer "B.Cu") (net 6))
 (segment (start 141.6304 88.3412) (end 139.4968 88.3412) (width 0.25) (layer "B.Cu") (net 6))
 (segment (start 139.4968 88.3412) (end 138.7348 87.5792) (width 0.25) (layer "B.Cu") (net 6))
 (segment (start 136.0932 87.5792) (end 135.815002 87.301002) (width 0.25) (layer "B.Cu") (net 6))
 (segment (start 135.815002 87.301002) (end 135.815002 86.233) (width 0.25) (layer "B.Cu") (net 6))
 (segment (start 144.145 91.297) (end 144.923 92.075) (width 0.25) (layer "F.Cu") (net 13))
 (segment (start 144.145 91.059) (end 144.145 91.297) (width 0.25) (layer "F.Cu") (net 13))
 (via (at 144.145 91.059) (size 0.6) (drill 0.3) (layers "F.Cu" "B.Cu") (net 13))
 (segment (start 141.5796 87.3252) (end 142.7988 87.3252) (width 0.25) (layer "B.Cu") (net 13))
 (segment (start 139.043691 87.126091) (end 139.794523 87.876923) (width 0.25) (layer "B.Cu") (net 13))
 (segment (start 139.794523 87.876923) (end 141.027877 87.876923) (width 0.25) (layer "B.Cu") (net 13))
 (segment (start 143.2814 87.8078) (end 143.2814 90.1954) (width 0.25) (layer "B.Cu") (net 13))
 (segment (start 141.027877 87.876923) (end 141.5796 87.3252) (width 0.25) (layer "B.Cu") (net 13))
 (segment (start 136.465 86.233) (end 136.465 86.808) (width 0.25) (layer "B.Cu") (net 13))
 (segment (start 136.465 86.808) (end 136.749509 87.126091) (width 0.25) (layer "B.Cu") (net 13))
 (segment (start 142.7988 87.3252) (end 143.2814 87.8078) (width 0.25) (layer "B.Cu") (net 13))
 (segment (start 136.749509 87.126091) (end 139.043691 87.126091) (width 0.25) (layer "B.Cu") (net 13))
 (segment (start 143.2814 90.1954) (end 144.145 91.059) (width 0.25) (layer "B.Cu") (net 13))
 (segment (start 146.948 92.05) (end 146.923 92.075) (width 0.25) (layer "F.Cu") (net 12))
 (segment (start 146.948 89.916) (end 146.948 92.05) (width 0.25) (layer "F.Cu") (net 12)))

